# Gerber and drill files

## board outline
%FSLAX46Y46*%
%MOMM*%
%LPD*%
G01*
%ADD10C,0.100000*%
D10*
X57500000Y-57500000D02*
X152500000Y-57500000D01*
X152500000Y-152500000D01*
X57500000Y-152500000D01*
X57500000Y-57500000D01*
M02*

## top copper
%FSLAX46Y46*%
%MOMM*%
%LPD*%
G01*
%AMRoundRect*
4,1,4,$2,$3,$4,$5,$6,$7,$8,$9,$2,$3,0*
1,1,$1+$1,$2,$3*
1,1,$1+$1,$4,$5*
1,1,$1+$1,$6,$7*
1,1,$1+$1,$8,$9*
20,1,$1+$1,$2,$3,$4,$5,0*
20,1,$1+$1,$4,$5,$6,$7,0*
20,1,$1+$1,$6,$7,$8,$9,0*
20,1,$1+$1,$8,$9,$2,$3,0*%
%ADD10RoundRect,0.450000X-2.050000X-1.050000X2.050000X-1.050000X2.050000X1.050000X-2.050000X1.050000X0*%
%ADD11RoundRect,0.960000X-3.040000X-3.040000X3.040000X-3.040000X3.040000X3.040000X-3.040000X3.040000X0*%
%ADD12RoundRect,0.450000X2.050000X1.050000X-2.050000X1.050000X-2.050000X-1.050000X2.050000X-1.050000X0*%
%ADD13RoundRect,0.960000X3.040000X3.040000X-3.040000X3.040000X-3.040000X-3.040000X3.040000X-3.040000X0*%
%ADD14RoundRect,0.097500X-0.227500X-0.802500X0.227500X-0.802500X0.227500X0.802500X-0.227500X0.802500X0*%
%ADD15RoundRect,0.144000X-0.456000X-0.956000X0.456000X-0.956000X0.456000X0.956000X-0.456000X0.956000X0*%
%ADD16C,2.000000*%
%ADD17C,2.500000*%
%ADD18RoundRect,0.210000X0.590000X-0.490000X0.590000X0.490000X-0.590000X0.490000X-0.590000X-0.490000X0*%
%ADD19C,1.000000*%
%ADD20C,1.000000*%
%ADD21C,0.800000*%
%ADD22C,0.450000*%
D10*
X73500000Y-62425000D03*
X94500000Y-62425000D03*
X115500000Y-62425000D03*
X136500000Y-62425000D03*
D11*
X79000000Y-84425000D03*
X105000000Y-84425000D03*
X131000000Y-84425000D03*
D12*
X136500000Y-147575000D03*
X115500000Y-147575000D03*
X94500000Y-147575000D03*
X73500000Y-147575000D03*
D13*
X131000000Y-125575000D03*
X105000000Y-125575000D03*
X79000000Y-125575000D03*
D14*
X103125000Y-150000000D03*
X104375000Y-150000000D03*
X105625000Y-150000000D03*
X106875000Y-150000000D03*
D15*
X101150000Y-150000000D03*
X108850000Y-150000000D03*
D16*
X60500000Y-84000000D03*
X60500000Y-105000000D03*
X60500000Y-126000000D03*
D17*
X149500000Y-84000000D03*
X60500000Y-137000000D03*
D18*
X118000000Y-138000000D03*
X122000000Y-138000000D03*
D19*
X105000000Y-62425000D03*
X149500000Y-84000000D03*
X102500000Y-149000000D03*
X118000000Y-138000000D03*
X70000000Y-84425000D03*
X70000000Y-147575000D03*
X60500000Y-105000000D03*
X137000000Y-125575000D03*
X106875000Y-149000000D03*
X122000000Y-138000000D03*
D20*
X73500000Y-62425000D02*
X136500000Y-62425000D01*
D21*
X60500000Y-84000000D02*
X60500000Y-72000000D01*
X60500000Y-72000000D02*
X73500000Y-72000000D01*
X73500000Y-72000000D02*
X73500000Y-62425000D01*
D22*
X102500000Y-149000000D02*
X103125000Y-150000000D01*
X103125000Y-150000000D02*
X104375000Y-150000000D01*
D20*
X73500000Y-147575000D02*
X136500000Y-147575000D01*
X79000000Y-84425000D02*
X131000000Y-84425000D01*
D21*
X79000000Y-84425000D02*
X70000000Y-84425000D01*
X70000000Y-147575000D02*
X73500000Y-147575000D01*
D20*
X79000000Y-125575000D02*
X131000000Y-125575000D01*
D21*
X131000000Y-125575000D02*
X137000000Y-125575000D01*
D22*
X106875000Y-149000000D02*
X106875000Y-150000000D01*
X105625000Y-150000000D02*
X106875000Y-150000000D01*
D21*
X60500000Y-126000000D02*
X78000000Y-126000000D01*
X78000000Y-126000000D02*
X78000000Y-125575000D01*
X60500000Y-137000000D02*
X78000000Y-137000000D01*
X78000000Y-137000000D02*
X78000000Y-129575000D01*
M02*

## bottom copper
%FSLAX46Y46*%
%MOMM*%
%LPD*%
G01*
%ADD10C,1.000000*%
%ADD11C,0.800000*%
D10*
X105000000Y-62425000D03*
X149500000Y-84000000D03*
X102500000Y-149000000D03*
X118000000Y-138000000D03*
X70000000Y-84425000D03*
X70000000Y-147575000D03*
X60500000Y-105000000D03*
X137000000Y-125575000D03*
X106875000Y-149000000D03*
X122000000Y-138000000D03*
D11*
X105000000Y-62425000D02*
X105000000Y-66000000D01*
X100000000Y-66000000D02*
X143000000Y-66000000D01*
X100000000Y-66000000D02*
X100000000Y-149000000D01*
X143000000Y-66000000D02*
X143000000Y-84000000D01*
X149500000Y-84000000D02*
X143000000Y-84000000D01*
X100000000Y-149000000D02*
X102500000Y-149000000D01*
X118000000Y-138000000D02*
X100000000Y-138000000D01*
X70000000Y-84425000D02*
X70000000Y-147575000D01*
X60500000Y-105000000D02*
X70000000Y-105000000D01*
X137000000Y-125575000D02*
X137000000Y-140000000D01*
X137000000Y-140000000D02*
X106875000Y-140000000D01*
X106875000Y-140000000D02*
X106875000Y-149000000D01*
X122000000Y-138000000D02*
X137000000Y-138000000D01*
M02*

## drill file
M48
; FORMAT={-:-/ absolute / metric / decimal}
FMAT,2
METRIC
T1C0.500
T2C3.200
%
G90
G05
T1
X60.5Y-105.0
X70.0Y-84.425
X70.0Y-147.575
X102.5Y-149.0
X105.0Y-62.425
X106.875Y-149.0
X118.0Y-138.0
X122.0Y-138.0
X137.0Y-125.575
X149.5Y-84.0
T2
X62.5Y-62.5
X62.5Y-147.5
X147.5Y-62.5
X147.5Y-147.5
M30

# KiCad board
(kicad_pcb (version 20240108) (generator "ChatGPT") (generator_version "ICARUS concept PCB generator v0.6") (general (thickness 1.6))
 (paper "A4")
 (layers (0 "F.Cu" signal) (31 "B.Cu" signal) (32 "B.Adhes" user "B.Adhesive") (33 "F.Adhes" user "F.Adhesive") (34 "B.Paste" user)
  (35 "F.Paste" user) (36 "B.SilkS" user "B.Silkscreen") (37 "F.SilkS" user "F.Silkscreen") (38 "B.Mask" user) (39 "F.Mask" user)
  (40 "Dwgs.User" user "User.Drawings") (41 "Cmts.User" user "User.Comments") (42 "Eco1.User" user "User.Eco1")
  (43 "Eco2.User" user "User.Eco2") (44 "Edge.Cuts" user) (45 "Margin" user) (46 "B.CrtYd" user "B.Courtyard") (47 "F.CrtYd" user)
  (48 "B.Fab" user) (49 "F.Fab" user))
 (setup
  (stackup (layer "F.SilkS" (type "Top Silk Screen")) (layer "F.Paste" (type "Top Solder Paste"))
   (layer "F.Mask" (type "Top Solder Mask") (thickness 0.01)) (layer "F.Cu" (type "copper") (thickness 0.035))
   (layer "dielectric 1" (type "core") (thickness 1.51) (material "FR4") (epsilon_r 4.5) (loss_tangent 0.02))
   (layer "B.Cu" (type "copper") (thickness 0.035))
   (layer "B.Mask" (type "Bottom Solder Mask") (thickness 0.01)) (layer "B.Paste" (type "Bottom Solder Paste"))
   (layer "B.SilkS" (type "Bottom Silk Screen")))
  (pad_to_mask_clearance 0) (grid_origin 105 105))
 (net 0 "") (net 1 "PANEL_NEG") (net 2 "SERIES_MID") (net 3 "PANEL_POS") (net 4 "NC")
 (gr_rect (start 57.5 57.5) (end 152.5 152.5) (stroke (width 0.1) (type solid)) (fill none) (layer "Edge.Cuts"))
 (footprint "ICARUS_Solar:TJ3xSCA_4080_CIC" (layer "F.Cu") (at 105 84.425 0)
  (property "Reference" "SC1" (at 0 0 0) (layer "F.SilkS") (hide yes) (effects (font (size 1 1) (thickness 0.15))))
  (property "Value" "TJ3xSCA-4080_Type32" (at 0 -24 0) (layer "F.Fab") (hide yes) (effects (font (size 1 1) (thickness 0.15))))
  (pad "1" smd roundrect (at -31.5 -22.0) (size 5.0 3.0) (layers "F.Cu" "F.Mask" "F.Paste") (roundrect_rratio 0.15) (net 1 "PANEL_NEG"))
  (pad "1" smd roundrect (at -10.5 -22.0) (size 5.0 3.0) (layers "F.Cu" "F.Mask" "F.Paste") (roundrect_rratio 0.15) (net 1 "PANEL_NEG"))
  (pad "1" smd roundrect (at 10.5 -22.0) (size 5.0 3.0) (layers "F.Cu" "F.Mask" "F.Paste") (roundrect_rratio 0.15) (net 1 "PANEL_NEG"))
  (pad "1" smd roundrect (at 31.5 -22.0) (size 5.0 3.0) (layers "F.Cu" "F.Mask" "F.Paste") (roundrect_rratio 0.15) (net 1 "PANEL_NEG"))
  (pad "2" smd roundrect (at -26.0 0) (size 8.0 8.0) (layers "F.Cu" "F.Mask") (roundrect_rratio 0.12) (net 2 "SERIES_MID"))
  (pad "2" smd roundrect (at 0 0) (size 8.0 8.0) (layers "F.Cu" "F.Mask") (roundrect_rratio 0.12) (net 2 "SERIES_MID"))
  (pad "2" smd roundrect (at 26.0 0) (size 8.0 8.0) (layers "F.Cu" "F.Mask") (roundrect_rratio 0.12) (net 2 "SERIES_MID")))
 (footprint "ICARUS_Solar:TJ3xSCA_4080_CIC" (layer "F.Cu") (at 105 125.575 180)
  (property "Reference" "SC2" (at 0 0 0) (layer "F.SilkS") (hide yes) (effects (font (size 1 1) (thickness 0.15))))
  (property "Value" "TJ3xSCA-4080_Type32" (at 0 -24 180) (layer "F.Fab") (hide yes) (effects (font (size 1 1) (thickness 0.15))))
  (pad "1" smd roundrect (at -31.5 -22.0 180) (size 5.0 3.0) (layers "F.Cu" "F.Mask" "F.Paste") (roundrect_rratio 0.15) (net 2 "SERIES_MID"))
  (pad "1" smd roundrect (at -10.5 -22.0 180) (size 5.0 3.0) (layers "F.Cu" "F.Mask" "F.Paste") (roundrect_rratio 0.15) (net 2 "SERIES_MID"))
  (pad "1" smd roundrect (at 10.5 -22.0 180) (size 5.0 3.0) (layers "F.Cu" "F.Mask" "F.Paste") (roundrect_rratio 0.15) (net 2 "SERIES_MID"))
  (pad "1" smd roundrect (at 31.5 -22.0 180) (size 5.0 3.0) (layers "F.Cu" "F.Mask" "F.Paste") (roundrect_rratio 0.15) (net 2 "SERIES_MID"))
  (pad "2" smd roundrect (at -26.0 0 180) (size 8.0 8.0) (layers "F.Cu" "F.Mask") (roundrect_rratio 0.12) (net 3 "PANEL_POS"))
  (pad "2" smd roundrect (at 0 0 180) (size 8.0 8.0) (layers "F.Cu" "F.Mask") (roundrect_rratio 0.12) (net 3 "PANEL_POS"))
  (pad "2" smd roundrect (at 26.0 0 180) (size 8.0 8.0) (layers "F.Cu" "F.Mask") (roundrect_rratio 0.12) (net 3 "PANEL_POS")))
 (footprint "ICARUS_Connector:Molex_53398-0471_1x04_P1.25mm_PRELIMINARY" (layer "F.Cu") (at 105 150 0)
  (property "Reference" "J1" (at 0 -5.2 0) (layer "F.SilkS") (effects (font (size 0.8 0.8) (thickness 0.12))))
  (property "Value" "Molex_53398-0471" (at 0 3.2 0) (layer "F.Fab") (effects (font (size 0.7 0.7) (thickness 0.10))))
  (pad "1" smd roundrect (at -1.875 0) (size 0.65 1.8) (layers "F.Cu" "F.Mask" "F.Paste") (roundrect_rratio 0.15) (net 1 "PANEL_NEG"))
  (pad "2" smd roundrect (at -0.625 0) (size 0.65 1.8) (layers "F.Cu" "F.Mask" "F.Paste") (roundrect_rratio 0.15) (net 1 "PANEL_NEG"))
  (pad "3" smd roundrect (at 0.625 0) (size 0.65 1.8) (layers "F.Cu" "F.Mask" "F.Paste") (roundrect_rratio 0.15) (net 3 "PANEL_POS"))
  (pad "4" smd roundrect (at 1.875 0) (size 0.65 1.8) (layers "F.Cu" "F.Mask" "F.Paste") (roundrect_rratio 0.15) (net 3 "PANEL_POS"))
  (pad "MP1" smd roundrect (at -3.85 0) (size 1.2 2.2) (layers "F.Cu" "F.Mask" "F.Paste") (roundrect_rratio 0.12))
  (pad "MP2" smd roundrect (at 3.85 0) (size 1.2 2.2) (layers "F.Cu" "F.Mask" "F.Paste") (roundrect_rratio 0.12)))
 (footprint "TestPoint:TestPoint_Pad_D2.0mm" (layer "F.Cu") (at 60.5 84 0)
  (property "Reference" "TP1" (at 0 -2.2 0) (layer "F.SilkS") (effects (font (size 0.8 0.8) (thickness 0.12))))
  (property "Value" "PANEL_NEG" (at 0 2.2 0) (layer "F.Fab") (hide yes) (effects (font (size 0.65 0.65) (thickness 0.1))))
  (pad "1" smd circle (at 0 0) (size 2.0 2.0) (layers "F.Cu" "F.Mask") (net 1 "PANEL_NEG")))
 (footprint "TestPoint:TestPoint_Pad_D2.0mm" (layer "F.Cu") (at 60.5 105 0)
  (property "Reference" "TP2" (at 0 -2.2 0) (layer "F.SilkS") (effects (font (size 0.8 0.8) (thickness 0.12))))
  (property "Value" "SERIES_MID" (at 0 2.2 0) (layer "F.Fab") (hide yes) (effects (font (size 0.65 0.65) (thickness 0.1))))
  (pad "1" smd circle (at 0 0) (size 2.0 2.0) (layers "F.Cu" "F.Mask") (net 2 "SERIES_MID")))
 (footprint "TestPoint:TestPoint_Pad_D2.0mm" (layer "F.Cu") (at 60.5 126 0)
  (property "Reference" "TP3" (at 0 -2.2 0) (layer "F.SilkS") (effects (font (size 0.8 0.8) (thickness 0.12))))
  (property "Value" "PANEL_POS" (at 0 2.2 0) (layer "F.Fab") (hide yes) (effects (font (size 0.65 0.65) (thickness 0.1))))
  (pad "1" smd circle (at 0 0) (size 2.0 2.0) (layers "F.Cu" "F.Mask") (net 3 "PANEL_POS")))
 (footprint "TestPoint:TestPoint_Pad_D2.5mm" (layer "F.Cu") (at 149.5 84 0)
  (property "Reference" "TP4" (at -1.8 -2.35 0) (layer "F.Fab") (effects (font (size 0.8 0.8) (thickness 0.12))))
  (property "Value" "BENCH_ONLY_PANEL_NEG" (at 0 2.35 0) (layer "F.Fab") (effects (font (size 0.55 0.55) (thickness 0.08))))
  (pad "1" smd circle (at 0 0) (size 2.5 2.5) (layers "F.Cu" "F.Mask") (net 1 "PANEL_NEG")))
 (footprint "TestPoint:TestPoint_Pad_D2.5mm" (layer "F.Cu") (at 60.5 137 0)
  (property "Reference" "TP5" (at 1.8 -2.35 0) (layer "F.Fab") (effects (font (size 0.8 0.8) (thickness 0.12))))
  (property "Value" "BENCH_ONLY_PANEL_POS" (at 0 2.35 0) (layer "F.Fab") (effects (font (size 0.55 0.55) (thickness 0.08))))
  (pad "1" smd circle (at 0 0) (size 2.5 2.5) (layers "F.Cu" "F.Mask") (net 3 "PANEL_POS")))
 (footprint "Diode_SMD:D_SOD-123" (layer "F.Cu") (at 120 138 0)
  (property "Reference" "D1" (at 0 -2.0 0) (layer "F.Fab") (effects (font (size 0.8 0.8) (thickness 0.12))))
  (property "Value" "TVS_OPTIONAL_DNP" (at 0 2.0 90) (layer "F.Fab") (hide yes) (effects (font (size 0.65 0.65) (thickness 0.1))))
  (pad "1" smd roundrect (at -2.0 0 90) (size 1.4 1.6) (layers "F.Cu" "F.Mask" "F.Paste") (roundrect_rratio 0.15) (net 1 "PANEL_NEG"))
  (pad "2" smd roundrect (at 2.0 0 90) (size 1.4 1.6) (layers "F.Cu" "F.Mask" "F.Paste") (roundrect_rratio 0.15) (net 3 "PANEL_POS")))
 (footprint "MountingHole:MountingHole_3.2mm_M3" (layer "F.Cu") (at 62.5 62.5)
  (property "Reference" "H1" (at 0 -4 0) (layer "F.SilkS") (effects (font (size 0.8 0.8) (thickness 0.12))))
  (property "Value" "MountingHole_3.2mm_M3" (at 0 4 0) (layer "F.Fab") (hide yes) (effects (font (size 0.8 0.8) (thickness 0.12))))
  (pad "" np_thru_hole circle (at 0 0) (size 3.2 3.2) (drill 3.2) (layers "*.Cu" "*.Mask")))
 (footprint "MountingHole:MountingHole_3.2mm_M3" (layer "F.Cu") (at 147.5 62.5)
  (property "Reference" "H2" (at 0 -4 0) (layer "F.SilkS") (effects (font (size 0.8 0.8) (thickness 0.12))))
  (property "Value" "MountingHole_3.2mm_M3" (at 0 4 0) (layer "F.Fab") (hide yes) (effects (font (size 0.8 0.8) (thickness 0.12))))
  (pad "" np_thru_hole circle (at 0 0) (size 3.2 3.2) (drill 3.2) (layers "*.Cu" "*.Mask")))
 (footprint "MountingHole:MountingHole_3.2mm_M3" (layer "F.Cu") (at 62.5 147.5)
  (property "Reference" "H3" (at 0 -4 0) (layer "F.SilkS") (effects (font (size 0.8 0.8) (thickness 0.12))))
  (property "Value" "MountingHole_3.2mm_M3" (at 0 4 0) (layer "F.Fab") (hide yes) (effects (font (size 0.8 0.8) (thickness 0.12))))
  (pad "" np_thru_hole circle (at 0 0) (size 3.2 3.2) (drill 3.2) (layers "*.Cu" "*.Mask")))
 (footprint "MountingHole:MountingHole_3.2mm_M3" (layer "F.Cu") (at 147.5 147.5)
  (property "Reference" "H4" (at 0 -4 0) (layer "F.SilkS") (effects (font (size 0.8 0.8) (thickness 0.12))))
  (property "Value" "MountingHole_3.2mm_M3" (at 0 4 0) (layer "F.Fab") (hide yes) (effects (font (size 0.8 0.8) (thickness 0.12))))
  (pad "" np_thru_hole circle (at 0 0) (size 3.2 3.2) (drill 3.2) (layers "*.Cu" "*.Mask")))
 (segment (start 73.5 62.425) (end 136.5 62.425) (width 1.0) (layer "F.Cu") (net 1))
 (segment (start 60.5 84) (end 60.5 72) (width 0.8) (layer "F.Cu") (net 1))
 (segment (start 60.5 72) (end 73.5 72) (width 0.8) (layer "F.Cu") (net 1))
 (segment (start 73.5 72) (end 73.5 62.425) (width 0.8) (layer "F.Cu") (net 1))
 (via (at 105 62.425) (size 1.0) (drill 0.5) (layers "F.Cu" "B.Cu") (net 1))
 (segment (start 105 62.425) (end 105 66) (width 0.8) (layer "B.Cu") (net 1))
 (segment (start 100 66) (end 143 66) (width 0.8) (layer "B.Cu") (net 1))
 (segment (start 100 66) (end 100 149) (width 0.8) (layer "B.Cu") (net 1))
 (segment (start 143 66) (end 143 84) (width 0.8) (layer "B.Cu") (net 1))
 (via (at 149.5 84) (size 1.0) (drill 0.5) (layers "F.Cu" "B.Cu") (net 1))
 (segment (start 149.5 84) (end 143 84) (width 0.8) (layer "B.Cu") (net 1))
 (segment (start 100 149) (end 102.5 149) (width 0.8) (layer "B.Cu") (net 1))
 (via (at 102.5 149) (size 1.0) (drill 0.5) (layers "F.Cu" "B.Cu") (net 1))
 (segment (start 102.5 149) (end 103.125 150) (width 0.45) (layer "F.Cu") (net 1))
 (segment (start 103.125 150) (end 104.375 150) (width 0.45) (layer "F.Cu") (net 1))
 (via (at 118 138) (size 1.0) (drill 0.5) (layers "F.Cu" "B.Cu") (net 1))
 (segment (start 118 138) (end 100 138) (width 0.8) (layer "B.Cu") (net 1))
 (segment (start 73.5 147.575) (end 136.5 147.575) (width 1.0) (layer "F.Cu") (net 2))
 (segment (start 79 84.425) (end 131 84.425) (width 1.0) (layer "F.Cu") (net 2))
 (segment (start 79 84.425) (end 70 84.425) (width 0.8) (layer "F.Cu") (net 2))
 (via (at 70 84.425) (size 1.0) (drill 0.5) (layers "F.Cu" "B.Cu") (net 2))
 (segment (start 70 84.425) (end 70 147.575) (width 0.8) (layer "B.Cu") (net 2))
 (via (at 70 147.575) (size 1.0) (drill 0.5) (layers "F.Cu" "B.Cu") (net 2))
 (segment (start 70 147.575) (end 73.5 147.575) (width 0.8) (layer "F.Cu") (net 2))
 (via (at 60.5 105) (size 1.0) (drill 0.5) (layers "F.Cu" "B.Cu") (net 2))
 (segment (start 60.5 105) (end 70 105) (width 0.8) (layer "B.Cu") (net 2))
 (segment (start 79 125.575) (end 131 125.575) (width 1.0) (layer "F.Cu") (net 3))
 (segment (start 131 125.575) (end 137 125.575) (width 0.8) (layer "F.Cu") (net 3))
 (via (at 137 125.575) (size 1.0) (drill 0.5) (layers "F.Cu" "B.Cu") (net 3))
 (segment (start 137 125.575) (end 137 140) (width 0.8) (layer "B.Cu") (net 3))
 (segment (start 137 140) (end 106.875 140) (width 0.8) (layer "B.Cu") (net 3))
 (segment (start 106.875 140) (end 106.875 149) (width 0.8) (layer "B.Cu") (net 3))
 (via (at 106.875 149) (size 1.0) (drill 0.5) (layers "F.Cu" "B.Cu") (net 3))
 (segment (start 106.875 149) (end 106.875 150) (width 0.45) (layer "F.Cu") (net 3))
 (segment (start 105.625 150) (end 106.875 150) (width 0.45) (layer "F.Cu") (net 3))
 (segment (start 60.5 126) (end 78 126) (width 0.8) (layer "F.Cu") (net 3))
 (segment (start 78 126) (end 78 125.575) (width 0.8) (layer "F.Cu") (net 3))
 (segment (start 60.5 137) (end 78 137) (width 0.8) (layer "F.Cu") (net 3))
 (segment (start 78 137) (end 78 129.575) (width 0.8) (layer "F.Cu") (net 3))
 (via (at 122 138) (size 1.0) (drill 0.5) (layers "F.Cu" "B.Cu") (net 3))
 (segment (start 122 138) (end 137 138) (width 0.8) (layer "B.Cu") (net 3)))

